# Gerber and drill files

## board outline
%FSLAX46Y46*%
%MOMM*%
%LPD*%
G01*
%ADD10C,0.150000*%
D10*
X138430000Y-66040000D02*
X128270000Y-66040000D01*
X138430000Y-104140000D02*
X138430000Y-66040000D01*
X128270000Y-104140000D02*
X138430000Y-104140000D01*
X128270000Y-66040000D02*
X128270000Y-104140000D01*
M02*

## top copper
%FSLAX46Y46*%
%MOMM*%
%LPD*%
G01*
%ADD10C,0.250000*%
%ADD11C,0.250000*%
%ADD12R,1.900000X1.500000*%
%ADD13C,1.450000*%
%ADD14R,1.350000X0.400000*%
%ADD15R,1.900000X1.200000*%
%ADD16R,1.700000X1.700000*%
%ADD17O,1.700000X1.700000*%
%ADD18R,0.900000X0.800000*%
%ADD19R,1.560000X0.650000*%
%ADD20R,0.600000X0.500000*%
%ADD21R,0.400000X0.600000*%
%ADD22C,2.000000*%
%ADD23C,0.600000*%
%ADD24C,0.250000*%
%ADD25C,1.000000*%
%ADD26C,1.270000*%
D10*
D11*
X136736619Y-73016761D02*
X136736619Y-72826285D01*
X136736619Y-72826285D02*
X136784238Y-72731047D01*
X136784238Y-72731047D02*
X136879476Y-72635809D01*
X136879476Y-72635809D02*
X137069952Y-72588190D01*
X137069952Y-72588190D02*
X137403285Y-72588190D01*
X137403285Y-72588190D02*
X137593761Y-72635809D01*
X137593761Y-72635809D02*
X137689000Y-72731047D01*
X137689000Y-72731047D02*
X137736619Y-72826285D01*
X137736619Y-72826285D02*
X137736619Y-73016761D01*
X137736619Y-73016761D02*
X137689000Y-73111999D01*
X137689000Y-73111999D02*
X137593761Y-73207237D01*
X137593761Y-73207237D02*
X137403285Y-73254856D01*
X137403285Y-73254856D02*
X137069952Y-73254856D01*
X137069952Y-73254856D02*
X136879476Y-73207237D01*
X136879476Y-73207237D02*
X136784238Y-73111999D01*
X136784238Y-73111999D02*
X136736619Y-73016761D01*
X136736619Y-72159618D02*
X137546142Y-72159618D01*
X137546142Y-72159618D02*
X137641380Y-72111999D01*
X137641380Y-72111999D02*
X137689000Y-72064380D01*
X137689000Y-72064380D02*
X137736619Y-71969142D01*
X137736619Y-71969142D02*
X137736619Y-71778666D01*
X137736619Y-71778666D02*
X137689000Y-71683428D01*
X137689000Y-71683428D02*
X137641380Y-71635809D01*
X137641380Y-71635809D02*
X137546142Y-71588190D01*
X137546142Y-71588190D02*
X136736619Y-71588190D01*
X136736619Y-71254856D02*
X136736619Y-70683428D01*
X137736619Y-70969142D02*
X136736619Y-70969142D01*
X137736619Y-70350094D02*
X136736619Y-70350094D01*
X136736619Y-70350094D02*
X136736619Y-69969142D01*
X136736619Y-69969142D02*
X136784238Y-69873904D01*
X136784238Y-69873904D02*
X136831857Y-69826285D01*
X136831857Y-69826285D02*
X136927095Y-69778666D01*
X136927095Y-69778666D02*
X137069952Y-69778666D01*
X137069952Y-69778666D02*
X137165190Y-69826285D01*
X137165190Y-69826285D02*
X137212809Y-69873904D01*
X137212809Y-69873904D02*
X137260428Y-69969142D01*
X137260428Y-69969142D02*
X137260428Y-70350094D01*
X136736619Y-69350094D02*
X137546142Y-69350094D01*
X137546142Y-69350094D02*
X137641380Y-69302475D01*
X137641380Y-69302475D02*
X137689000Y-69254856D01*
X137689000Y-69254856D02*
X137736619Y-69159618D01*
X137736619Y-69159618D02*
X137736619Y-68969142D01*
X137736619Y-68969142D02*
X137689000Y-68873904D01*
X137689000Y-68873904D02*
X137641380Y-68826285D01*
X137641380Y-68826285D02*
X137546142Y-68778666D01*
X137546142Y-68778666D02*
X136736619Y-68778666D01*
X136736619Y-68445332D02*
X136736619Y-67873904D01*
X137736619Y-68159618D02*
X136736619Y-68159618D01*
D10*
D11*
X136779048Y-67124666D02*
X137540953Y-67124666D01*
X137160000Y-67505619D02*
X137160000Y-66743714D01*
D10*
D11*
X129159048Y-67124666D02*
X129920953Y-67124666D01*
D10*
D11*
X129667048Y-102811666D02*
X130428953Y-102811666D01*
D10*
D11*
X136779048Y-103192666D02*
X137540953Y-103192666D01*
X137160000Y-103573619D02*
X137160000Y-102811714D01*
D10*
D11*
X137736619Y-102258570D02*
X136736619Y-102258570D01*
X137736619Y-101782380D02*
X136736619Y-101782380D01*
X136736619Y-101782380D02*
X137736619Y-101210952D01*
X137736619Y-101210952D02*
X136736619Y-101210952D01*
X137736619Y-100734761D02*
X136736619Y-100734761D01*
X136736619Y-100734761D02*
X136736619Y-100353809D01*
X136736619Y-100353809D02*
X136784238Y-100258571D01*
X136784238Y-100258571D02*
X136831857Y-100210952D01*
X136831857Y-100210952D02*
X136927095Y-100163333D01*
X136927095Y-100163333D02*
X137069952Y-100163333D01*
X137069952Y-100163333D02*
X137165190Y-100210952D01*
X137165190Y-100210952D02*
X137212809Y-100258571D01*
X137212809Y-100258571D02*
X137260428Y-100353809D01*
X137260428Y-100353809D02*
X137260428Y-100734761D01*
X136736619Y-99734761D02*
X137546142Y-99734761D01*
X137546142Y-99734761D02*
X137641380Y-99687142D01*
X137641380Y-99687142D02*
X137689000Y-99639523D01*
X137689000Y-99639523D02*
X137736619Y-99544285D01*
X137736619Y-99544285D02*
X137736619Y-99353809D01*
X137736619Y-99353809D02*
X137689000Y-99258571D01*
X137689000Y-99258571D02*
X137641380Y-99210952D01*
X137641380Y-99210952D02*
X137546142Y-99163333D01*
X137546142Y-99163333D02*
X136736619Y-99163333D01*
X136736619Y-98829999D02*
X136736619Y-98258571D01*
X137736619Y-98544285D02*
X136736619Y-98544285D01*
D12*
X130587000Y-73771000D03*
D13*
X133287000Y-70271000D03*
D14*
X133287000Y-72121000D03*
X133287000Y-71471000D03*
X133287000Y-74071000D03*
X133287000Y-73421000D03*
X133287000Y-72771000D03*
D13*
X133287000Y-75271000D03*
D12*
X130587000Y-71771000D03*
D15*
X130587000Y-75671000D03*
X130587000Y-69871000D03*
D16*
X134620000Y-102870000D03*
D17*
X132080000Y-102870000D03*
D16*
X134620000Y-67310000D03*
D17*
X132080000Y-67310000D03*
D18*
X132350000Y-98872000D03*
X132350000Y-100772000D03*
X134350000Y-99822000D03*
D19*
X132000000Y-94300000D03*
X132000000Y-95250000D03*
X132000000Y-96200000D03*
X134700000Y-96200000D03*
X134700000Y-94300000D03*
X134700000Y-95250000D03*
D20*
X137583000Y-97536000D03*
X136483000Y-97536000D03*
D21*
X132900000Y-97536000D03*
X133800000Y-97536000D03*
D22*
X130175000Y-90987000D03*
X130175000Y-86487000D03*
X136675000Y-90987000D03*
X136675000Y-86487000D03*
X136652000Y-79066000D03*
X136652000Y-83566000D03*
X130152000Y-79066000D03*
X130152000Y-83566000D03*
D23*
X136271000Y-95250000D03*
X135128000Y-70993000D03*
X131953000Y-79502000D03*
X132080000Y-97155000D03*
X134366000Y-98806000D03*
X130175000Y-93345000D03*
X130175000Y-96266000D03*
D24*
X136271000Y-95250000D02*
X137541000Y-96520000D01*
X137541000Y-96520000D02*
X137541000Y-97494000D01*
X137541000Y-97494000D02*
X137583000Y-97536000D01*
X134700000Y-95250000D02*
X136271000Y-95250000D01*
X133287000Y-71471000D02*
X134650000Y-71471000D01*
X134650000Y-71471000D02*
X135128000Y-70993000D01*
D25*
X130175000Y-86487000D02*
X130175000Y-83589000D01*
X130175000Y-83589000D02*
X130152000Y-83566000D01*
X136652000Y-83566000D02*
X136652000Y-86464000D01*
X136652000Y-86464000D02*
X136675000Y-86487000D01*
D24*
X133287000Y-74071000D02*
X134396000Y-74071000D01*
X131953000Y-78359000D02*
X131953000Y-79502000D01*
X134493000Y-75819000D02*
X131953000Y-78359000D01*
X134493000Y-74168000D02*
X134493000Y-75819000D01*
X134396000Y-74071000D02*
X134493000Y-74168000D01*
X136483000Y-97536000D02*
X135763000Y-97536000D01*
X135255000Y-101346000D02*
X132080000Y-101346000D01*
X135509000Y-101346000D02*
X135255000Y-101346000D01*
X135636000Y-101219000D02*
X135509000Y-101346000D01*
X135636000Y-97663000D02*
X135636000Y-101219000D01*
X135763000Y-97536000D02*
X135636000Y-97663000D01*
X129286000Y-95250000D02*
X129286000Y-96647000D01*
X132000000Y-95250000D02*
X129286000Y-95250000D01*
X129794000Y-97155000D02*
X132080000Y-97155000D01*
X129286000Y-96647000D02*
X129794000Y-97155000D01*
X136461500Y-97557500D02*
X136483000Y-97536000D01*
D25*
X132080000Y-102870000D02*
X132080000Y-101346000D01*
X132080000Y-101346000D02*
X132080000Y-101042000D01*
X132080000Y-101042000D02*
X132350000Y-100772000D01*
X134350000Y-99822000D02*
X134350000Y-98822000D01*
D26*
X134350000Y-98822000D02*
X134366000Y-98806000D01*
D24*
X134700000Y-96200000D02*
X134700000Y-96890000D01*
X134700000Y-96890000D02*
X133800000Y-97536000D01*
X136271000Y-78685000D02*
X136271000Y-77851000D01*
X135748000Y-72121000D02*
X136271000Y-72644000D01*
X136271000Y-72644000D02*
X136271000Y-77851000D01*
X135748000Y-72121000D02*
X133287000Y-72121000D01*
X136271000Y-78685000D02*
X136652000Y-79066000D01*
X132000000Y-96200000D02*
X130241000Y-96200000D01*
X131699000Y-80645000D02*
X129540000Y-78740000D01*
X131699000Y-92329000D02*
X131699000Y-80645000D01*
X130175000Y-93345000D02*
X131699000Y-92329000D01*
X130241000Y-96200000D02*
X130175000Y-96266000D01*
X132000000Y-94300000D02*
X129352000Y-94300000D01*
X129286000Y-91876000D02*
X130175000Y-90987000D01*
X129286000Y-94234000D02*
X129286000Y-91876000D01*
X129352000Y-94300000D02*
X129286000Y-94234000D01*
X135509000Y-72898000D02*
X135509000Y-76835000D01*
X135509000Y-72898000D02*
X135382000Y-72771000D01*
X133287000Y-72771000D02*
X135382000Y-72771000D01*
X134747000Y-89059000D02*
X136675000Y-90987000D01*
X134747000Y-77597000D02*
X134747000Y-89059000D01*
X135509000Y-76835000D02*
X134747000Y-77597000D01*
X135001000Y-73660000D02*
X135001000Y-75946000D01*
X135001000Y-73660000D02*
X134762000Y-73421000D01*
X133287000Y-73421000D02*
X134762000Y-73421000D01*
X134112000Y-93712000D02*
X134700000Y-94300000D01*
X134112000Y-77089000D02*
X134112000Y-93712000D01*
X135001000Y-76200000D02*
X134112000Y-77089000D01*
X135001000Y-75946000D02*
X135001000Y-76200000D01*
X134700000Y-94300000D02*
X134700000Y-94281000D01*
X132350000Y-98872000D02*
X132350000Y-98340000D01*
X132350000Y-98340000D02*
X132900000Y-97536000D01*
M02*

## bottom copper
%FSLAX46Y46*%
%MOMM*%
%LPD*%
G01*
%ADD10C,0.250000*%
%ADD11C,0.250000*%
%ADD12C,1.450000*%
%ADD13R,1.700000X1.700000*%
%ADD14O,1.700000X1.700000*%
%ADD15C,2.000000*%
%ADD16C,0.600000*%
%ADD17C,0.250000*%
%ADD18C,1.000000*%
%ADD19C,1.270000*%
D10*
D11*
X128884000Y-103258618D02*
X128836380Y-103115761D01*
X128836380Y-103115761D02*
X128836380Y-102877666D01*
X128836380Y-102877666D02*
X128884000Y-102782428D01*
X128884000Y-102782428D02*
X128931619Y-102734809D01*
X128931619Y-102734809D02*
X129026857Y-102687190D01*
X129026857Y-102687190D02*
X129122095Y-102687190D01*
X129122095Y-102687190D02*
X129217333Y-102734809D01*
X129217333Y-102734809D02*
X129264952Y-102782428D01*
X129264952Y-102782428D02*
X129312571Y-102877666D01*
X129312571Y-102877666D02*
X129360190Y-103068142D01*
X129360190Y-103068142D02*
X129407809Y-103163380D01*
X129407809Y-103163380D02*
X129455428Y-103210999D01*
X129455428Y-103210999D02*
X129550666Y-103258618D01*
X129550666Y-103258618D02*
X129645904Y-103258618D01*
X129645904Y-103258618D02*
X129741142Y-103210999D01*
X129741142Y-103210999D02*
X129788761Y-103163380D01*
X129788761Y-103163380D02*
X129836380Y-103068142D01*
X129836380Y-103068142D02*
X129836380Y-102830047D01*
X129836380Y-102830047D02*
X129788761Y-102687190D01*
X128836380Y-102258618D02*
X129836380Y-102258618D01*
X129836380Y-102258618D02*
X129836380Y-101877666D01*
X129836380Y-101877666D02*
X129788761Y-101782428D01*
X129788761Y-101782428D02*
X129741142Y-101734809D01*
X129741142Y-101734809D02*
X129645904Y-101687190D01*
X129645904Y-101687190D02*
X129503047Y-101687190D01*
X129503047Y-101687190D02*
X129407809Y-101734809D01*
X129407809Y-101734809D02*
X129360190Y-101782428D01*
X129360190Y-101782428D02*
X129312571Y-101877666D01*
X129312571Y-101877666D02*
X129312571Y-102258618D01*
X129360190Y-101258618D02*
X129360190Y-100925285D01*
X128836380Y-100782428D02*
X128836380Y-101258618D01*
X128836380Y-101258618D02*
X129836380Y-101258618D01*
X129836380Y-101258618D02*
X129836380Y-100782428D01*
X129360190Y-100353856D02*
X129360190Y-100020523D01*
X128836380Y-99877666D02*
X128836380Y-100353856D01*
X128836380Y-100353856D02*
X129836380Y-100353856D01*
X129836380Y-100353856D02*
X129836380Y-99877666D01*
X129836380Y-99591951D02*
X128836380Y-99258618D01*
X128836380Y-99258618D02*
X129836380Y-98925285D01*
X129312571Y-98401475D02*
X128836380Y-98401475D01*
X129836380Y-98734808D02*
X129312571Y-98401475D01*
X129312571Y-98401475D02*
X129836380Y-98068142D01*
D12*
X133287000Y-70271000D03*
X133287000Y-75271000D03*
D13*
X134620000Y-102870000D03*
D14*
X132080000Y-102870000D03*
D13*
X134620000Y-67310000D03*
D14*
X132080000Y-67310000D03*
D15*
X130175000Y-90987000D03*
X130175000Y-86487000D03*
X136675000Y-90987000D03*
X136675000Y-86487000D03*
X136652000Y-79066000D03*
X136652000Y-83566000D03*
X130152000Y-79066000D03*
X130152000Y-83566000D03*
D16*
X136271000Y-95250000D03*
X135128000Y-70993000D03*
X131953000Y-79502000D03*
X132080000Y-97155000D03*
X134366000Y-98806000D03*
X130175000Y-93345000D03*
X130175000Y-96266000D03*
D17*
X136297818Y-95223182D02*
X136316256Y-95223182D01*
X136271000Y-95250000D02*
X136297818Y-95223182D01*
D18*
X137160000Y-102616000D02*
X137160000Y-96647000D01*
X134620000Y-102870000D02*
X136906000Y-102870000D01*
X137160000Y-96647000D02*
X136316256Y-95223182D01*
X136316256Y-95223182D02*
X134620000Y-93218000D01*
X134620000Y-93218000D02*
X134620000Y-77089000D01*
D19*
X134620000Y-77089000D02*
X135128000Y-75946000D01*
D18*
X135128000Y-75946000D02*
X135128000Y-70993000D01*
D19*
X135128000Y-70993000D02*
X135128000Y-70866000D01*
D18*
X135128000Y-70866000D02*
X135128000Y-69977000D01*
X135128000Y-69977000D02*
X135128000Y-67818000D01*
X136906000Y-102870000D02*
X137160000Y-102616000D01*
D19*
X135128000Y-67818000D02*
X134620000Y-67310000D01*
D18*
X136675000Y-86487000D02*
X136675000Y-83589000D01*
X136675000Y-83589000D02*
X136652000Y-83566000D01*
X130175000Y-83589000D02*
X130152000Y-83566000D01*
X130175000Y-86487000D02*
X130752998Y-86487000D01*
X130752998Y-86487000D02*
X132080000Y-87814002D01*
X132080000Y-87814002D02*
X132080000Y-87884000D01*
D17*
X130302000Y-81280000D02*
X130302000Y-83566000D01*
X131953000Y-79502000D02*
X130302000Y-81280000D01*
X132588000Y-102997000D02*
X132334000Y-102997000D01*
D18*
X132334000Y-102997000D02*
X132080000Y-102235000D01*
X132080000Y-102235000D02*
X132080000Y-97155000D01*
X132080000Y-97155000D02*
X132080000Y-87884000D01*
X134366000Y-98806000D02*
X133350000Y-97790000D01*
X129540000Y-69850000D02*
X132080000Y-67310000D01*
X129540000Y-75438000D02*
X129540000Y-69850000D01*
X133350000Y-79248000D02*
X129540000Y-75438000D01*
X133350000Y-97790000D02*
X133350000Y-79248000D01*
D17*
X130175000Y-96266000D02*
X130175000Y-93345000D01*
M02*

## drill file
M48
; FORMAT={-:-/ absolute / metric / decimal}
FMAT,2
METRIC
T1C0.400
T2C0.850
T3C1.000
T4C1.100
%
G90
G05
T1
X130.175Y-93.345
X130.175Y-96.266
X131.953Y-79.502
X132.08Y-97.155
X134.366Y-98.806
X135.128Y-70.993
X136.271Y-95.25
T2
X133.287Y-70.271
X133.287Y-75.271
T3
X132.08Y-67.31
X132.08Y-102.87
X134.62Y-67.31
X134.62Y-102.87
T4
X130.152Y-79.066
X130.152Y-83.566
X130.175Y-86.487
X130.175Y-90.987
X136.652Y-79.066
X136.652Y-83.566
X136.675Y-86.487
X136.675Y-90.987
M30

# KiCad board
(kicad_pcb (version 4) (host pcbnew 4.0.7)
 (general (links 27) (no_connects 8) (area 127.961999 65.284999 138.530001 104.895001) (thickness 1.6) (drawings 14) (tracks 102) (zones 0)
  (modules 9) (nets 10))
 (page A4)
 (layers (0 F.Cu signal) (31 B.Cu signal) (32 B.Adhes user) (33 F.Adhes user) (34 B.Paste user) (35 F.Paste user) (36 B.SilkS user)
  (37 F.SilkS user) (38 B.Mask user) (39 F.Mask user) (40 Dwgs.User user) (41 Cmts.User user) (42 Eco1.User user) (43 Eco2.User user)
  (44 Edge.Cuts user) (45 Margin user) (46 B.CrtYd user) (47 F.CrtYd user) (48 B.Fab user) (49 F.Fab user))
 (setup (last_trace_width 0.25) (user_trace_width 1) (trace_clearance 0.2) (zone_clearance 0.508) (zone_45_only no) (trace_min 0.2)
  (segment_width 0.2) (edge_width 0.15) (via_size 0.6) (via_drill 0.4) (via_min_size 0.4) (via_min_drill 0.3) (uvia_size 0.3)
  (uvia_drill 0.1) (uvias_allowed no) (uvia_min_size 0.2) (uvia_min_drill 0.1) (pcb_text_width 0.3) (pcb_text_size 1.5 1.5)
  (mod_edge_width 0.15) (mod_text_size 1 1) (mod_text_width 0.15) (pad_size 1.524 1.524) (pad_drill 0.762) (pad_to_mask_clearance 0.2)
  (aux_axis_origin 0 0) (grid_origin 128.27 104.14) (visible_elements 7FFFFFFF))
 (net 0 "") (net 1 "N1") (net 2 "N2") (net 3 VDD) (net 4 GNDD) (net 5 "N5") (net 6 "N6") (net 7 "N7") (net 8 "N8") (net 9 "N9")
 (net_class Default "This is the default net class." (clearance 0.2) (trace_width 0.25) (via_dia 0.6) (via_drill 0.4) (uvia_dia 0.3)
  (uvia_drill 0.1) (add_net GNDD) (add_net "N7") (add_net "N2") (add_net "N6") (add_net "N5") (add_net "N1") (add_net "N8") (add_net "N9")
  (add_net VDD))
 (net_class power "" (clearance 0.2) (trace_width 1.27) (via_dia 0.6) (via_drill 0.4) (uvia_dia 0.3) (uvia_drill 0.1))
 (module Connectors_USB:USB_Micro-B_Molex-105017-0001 (layer F.Cu) (at 130.937 72.771 270)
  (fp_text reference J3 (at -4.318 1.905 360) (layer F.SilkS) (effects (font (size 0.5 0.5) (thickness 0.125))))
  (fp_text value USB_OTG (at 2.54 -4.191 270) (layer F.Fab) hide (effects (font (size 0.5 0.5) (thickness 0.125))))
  (pad 6 smd rect (at 1 0.35 270) (size 1.5 1.9) (layers F.Cu F.Paste F.Mask) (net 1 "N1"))
  (pad 6 thru_hole circle (at -2.5 -2.35 270) (size 1.45 1.45) (drill 0.85) (layers *.Cu *.Mask) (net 1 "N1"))
  (pad 2 smd rect (at -0.65 -2.35 270) (size 0.4 1.35) (layers F.Cu F.Paste F.Mask) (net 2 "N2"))
  (pad 1 smd rect (at -1.3 -2.35 270) (size 0.4 1.35) (layers F.Cu F.Paste F.Mask) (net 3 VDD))
  (pad 5 smd rect (at 1.3 -2.35 270) (size 0.4 1.35) (layers F.Cu F.Paste F.Mask) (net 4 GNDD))
  (pad 4 smd rect (at 0.65 -2.35 270) (size 0.4 1.35) (layers F.Cu F.Paste F.Mask) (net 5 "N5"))
  (pad 3 smd rect (at 0 -2.35 270) (size 0.4 1.35) (layers F.Cu F.Paste F.Mask) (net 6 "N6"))
  (pad 6 thru_hole circle (at 2.5 -2.35 270) (size 1.45 1.45) (drill 0.85) (layers *.Cu *.Mask) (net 1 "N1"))
  (pad 6 smd rect (at -1 0.35 270) (size 1.5 1.9) (layers F.Cu F.Paste F.Mask) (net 1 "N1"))
  (pad 6 smd rect (at 2.9 0.35 270) (size 1.2 1.9) (layers F.Cu F.Mask) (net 1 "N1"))
  (pad 6 smd rect (at -2.9 0.35 270) (size 1.2 1.9) (layers F.Cu F.Mask) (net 1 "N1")))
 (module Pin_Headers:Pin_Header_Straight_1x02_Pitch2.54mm (layer F.Cu) (at 134.62 102.87 270)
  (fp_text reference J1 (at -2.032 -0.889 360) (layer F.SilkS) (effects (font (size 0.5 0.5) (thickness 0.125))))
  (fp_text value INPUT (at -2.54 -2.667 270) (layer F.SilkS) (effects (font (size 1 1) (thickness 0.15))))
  (pad 1 thru_hole rect (at 0 0 270) (size 1.7 1.7) (drill 1) (layers *.Cu *.Mask) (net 3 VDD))
  (pad 2 thru_hole oval (at 0 2.54 270) (size 1.7 1.7) (drill 1) (layers *.Cu *.Mask) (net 4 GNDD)))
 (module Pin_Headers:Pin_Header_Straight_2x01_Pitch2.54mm (layer F.Cu) (at 134.62 67.31 180)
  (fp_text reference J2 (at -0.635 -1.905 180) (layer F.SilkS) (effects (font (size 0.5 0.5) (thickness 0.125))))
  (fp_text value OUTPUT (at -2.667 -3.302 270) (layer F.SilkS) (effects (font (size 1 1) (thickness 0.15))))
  (pad 1 thru_hole rect (at 0 0 180) (size 1.7 1.7) (drill 1) (layers *.Cu *.Mask) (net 3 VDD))
  (pad 2 thru_hole oval (at 2.54 0 180) (size 1.7 1.7) (drill 1) (layers *.Cu *.Mask) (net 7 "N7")))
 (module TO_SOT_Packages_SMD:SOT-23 (layer F.Cu) (at 133.35 99.822)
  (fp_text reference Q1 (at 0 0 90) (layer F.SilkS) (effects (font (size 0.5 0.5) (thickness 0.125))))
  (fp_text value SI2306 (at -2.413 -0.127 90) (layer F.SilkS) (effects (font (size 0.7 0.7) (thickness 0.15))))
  (pad 1 smd rect (at -1 -0.95) (size 0.9 0.8) (layers F.Cu F.Paste F.Mask) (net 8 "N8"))
  (pad 2 smd rect (at -1 0.95) (size 0.9 0.8) (layers F.Cu F.Paste F.Mask) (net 4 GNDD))
  (pad 3 smd rect (at 1 0) (size 0.9 0.8) (layers F.Cu F.Paste F.Mask) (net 7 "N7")))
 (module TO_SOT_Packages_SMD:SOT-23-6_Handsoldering (layer F.Cu) (at 133.35 95.25)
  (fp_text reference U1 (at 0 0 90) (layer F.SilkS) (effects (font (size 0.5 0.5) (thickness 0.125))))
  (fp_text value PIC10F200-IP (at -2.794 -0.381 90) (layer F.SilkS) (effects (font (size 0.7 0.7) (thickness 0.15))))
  (pad 1 smd rect (at -1.35 -0.95) (size 1.56 0.65) (layers F.Cu F.Paste F.Mask) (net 6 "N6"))
  (pad 2 smd rect (at -1.35 0) (size 1.56 0.65) (layers F.Cu F.Paste F.Mask) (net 4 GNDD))
  (pad 3 smd rect (at -1.35 0.95) (size 1.56 0.65) (layers F.Cu F.Paste F.Mask) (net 2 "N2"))
  (pad 4 smd rect (at 1.35 0.95) (size 1.56 0.65) (layers F.Cu F.Paste F.Mask) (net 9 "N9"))
  (pad 6 smd rect (at 1.35 -0.95) (size 1.56 0.65) (layers F.Cu F.Paste F.Mask) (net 5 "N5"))
  (pad 5 smd rect (at 1.35 0) (size 1.56 0.65) (layers F.Cu F.Paste F.Mask) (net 3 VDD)))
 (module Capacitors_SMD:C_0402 (layer F.Cu) (at 137.033 97.536 180)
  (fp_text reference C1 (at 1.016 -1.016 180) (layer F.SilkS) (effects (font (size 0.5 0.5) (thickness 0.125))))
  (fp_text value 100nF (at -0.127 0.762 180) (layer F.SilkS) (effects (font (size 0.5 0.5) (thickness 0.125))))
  (pad 1 smd rect (at -0.55 0 180) (size 0.6 0.5) (layers F.Cu F.Paste F.Mask) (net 3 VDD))
  (pad 2 smd rect (at 0.55 0 180) (size 0.6 0.5) (layers F.Cu F.Paste F.Mask) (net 4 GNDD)))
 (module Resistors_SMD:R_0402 (layer F.Cu) (at 133.35 97.536)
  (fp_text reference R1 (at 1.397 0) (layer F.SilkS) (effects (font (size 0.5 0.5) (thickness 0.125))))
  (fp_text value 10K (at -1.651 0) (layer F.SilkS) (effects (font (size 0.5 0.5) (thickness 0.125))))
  (pad 1 smd rect (at -0.45 0) (size 0.4 0.6) (layers F.Cu F.Paste F.Mask) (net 8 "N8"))
  (pad 2 smd rect (at 0.45 0) (size 0.4 0.6) (layers F.Cu F.Paste F.Mask) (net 9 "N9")))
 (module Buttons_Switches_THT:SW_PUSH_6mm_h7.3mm (layer F.Cu) (at 130.175 86.487)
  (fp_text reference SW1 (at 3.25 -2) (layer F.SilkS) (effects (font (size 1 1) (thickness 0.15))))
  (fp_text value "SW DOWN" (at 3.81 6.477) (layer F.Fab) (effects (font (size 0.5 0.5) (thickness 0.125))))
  (pad 2 thru_hole circle (at 0 4.5 90) (size 2 2) (drill 1.1) (layers *.Cu *.Mask) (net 6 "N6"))
  (pad 1 thru_hole circle (at 0 0 90) (size 2 2) (drill 1.1) (layers *.Cu *.Mask) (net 4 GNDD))
  (pad 2 thru_hole circle (at 6.5 4.5 90) (size 2 2) (drill 1.1) (layers *.Cu *.Mask) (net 6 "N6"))
  (pad 1 thru_hole circle (at 6.5 0 90) (size 2 2) (drill 1.1) (layers *.Cu *.Mask) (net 4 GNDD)))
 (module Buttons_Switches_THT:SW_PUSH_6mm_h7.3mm (layer F.Cu) (at 136.652 83.566 180)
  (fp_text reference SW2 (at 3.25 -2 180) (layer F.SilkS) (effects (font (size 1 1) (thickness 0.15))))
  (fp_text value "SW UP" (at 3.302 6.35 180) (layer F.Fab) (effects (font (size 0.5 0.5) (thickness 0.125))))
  (pad 2 thru_hole circle (at 0 4.5 270) (size 2 2) (drill 1.1) (layers *.Cu *.Mask) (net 2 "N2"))
  (pad 1 thru_hole circle (at 0 0 270) (size 2 2) (drill 1.1) (layers *.Cu *.Mask) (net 4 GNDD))
  (pad 2 thru_hole circle (at 6.5 4.5 270) (size 2 2) (drill 1.1) (layers *.Cu *.Mask) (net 2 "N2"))
  (pad 1 thru_hole circle (at 6.5 0 270) (size 2 2) (drill 1.1) (layers *.Cu *.Mask) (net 4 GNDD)))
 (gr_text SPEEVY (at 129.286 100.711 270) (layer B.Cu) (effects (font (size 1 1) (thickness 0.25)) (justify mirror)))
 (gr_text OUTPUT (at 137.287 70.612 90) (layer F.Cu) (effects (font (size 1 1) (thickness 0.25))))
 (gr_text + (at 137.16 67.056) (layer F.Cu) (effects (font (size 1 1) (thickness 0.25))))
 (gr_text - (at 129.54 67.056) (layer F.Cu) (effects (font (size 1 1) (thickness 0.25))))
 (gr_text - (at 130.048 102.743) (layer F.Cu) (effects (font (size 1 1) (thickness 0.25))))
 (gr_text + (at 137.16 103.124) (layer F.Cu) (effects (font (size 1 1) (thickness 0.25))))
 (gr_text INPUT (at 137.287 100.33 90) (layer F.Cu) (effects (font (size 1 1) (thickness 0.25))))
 (gr_line (start 138.43 66.04) (end 128.27 66.04) (angle 90) (layer Edge.Cuts) (width 0.15))
 (gr_line (start 138.43 104.14) (end 138.43 66.04) (angle 90) (layer Edge.Cuts) (width 0.15))
 (gr_line (start 128.27 104.14) (end 138.43 104.14) (angle 90) (layer Edge.Cuts) (width 0.15))
 (gr_line (start 128.27 66.04) (end 128.27 104.14) (angle 90) (layer Edge.Cuts) (width 0.15))
 (segment (start 136.271 95.25) (end 137.541 96.52) (width 0.25) (layer F.Cu) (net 3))
 (segment (start 137.541 96.52) (end 137.541 97.494) (width 0.25) (layer F.Cu) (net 3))
 (segment (start 137.541 97.494) (end 137.583 97.536) (width 0.25) (layer F.Cu) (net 3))
 (segment (start 134.7 95.25) (end 136.271 95.25) (width 0.25) (layer F.Cu) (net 3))
 (segment (start 136.297818 95.223182) (end 136.316256 95.223182) (width 0.25) (layer B.Cu) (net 3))
 (segment (start 136.271 95.25) (end 136.297818 95.223182) (width 0.25) (layer B.Cu) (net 3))
 (via (at 136.271 95.25) (size 0.6) (drill 0.4) (layers F.Cu B.Cu) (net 3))
 (segment (start 133.287 71.471) (end 134.65 71.471) (width 0.25) (layer F.Cu) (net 3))
 (via (at 135.128 70.993) (size 0.6) (drill 0.4) (layers F.Cu B.Cu) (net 3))
 (segment (start 134.65 71.471) (end 135.128 70.993) (width 0.25) (layer F.Cu) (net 3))
 (segment (start 137.16 102.616) (end 137.16 96.647) (width 1) (layer B.Cu) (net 3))
 (segment (start 134.62 102.87) (end 136.906 102.87) (width 1) (layer B.Cu) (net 3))
 (segment (start 137.16 96.647) (end 136.316256 95.223182) (width 1) (layer B.Cu) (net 3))
 (segment (start 136.316256 95.223182) (end 134.62 93.218) (width 1) (layer B.Cu) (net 3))
 (segment (start 134.62 93.218) (end 134.62 77.089) (width 1) (layer B.Cu) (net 3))
 (segment (start 134.62 77.089) (end 135.128 75.946) (width 1.27) (layer B.Cu) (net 3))
 (segment (start 135.128 75.946) (end 135.128 70.993) (width 1) (layer B.Cu) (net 3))
 (segment (start 135.128 70.993) (end 135.128 70.866) (width 1.27) (layer B.Cu) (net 3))
 (segment (start 135.128 70.866) (end 135.128 69.977) (width 1) (layer B.Cu) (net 3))
 (segment (start 135.128 69.977) (end 135.128 67.818) (width 1) (layer B.Cu) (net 3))
 (segment (start 136.906 102.87) (end 137.16 102.616) (width 1) (layer B.Cu) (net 3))
 (segment (start 135.128 67.818) (end 134.62 67.31) (width 1.27) (layer B.Cu) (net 3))
 (segment (start 130.175 86.487) (end 130.175 83.589) (width 1) (layer F.Cu) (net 4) (status C00000))
 (segment (start 130.175 83.589) (end 130.152 83.566) (width 1) (layer F.Cu) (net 4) (status C00000))
 (segment (start 136.652 83.566) (end 136.652 86.464) (width 1) (layer F.Cu) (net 4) (status C00000))
 (segment (start 136.652 86.464) (end 136.675 86.487) (width 1) (layer F.Cu) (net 4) (status C00000))
 (segment (start 136.675 86.487) (end 136.675 83.589) (width 1) (layer B.Cu) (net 4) (status C00000))
 (segment (start 136.675 83.589) (end 136.652 83.566) (width 1) (layer B.Cu) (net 4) (status C00000))
 (segment (start 130.175 83.589) (end 130.152 83.566) (width 1) (layer B.Cu) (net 4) (status C00000))
 (segment (start 130.175 86.487) (end 130.752998 86.487) (width 1) (layer B.Cu) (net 4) (status C00000))
 (segment (start 130.752998 86.487) (end 132.08 87.814002) (width 1) (layer B.Cu) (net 4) (status 400000))
 (segment (start 132.08 87.814002) (end 132.08 87.884) (width 1) (layer B.Cu) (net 4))
 (segment (start 133.287 74.071) (end 134.396 74.071) (width 0.25) (layer F.Cu) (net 4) (status 400000))
 (segment (start 130.302 81.28) (end 130.302 83.566) (width 0.25) (layer B.Cu) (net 4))
 (segment (start 131.953 79.502) (end 130.302 81.28) (width 0.25) (layer B.Cu) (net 4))
 (via (at 131.953 79.502) (size 0.6) (drill 0.4) (layers F.Cu B.Cu) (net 4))
 (segment (start 131.953 78.359) (end 131.953 79.502) (width 0.25) (layer F.Cu) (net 4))
 (segment (start 134.493 75.819) (end 131.953 78.359) (width 0.25) (layer F.Cu) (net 4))
 (segment (start 134.493 74.168) (end 134.493 75.819) (width 0.25) (layer F.Cu) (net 4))
 (segment (start 134.396 74.071) (end 134.493 74.168) (width 0.25) (layer F.Cu) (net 4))
 (segment (start 136.483 97.536) (end 135.763 97.536) (width 0.25) (layer F.Cu) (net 4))
 (segment (start 135.255 101.346) (end 132.08 101.346) (width 0.25) (layer F.Cu) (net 4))
 (segment (start 135.509 101.346) (end 135.255 101.346) (width 0.25) (layer F.Cu) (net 4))
 (segment (start 135.636 101.219) (end 135.509 101.346) (width 0.25) (layer F.Cu) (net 4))
 (segment (start 135.636 97.663) (end 135.636 101.219) (width 0.25) (layer F.Cu) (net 4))
 (segment (start 135.763 97.536) (end 135.636 97.663) (width 0.25) (layer F.Cu) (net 4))
 (segment (start 129.286 95.25) (end 129.286 96.647) (width 0.25) (layer F.Cu) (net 4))
 (segment (start 132 95.25) (end 129.286 95.25) (width 0.25) (layer F.Cu) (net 4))
 (via (at 132.08 97.155) (size 0.6) (drill 0.4) (layers F.Cu B.Cu) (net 4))
 (segment (start 129.794 97.155) (end 132.08 97.155) (width 0.25) (layer F.Cu) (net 4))
 (segment (start 129.286 96.647) (end 129.794 97.155) (width 0.25) (layer F.Cu) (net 4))
 (segment (start 132.588 102.997) (end 132.334 102.997) (width 0.25) (layer B.Cu) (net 4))
 (segment (start 132.334 102.997) (end 132.08 102.235) (width 1) (layer B.Cu) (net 4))
 (segment (start 132.08 102.235) (end 132.08 97.155) (width 1) (layer B.Cu) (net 4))
 (segment (start 132.08 97.155) (end 132.08 87.884) (width 1) (layer B.Cu) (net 4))
 (segment (start 136.4615 97.5575) (end 136.483 97.536) (width 0.25) (layer F.Cu) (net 4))
 (segment (start 132.08 102.87) (end 132.08 101.346) (width 1) (layer F.Cu) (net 4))
 (segment (start 132.08 101.346) (end 132.08 101.042) (width 1) (layer F.Cu) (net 4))
 (segment (start 132.08 101.042) (end 132.35 100.772) (width 1) (layer F.Cu) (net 4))
 (segment (start 134.366 98.806) (end 133.35 97.79) (width 1) (layer B.Cu) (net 7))
 (segment (start 134.35 99.822) (end 134.35 98.822) (width 1) (layer F.Cu) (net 7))
 (via (at 134.366 98.806) (size 0.6) (drill 0.4) (layers F.Cu B.Cu) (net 7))
 (segment (start 134.35 98.822) (end 134.366 98.806) (width 1.27) (layer F.Cu) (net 7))
 (segment (start 129.54 69.85) (end 132.08 67.31) (width 1) (layer B.Cu) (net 7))
 (segment (start 129.54 75.438) (end 129.54 69.85) (width 1) (layer B.Cu) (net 7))
 (segment (start 133.35 79.248) (end 129.54 75.438) (width 1) (layer B.Cu) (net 7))
 (segment (start 133.35 97.79) (end 133.35 79.248) (width 1) (layer B.Cu) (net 7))
 (segment (start 134.7 96.2) (end 134.7 96.89) (width 0.25) (layer F.Cu) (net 9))
 (segment (start 134.7 96.89) (end 133.8 97.536) (width 0.25) (layer F.Cu) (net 9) (status 20))
 (segment (start 136.271 78.685) (end 136.271 77.851) (width 0.25) (layer F.Cu) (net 2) (status 400000))
 (segment (start 135.748 72.121) (end 136.271 72.644) (width 0.25) (layer F.Cu) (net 2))
 (segment (start 136.271 72.644) (end 136.271 77.851) (width 0.25) (layer F.Cu) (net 2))
 (segment (start 135.748 72.121) (end 133.287 72.121) (width 0.25) (layer F.Cu) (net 2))
 (segment (start 136.271 78.685) (end 136.652 79.066) (width 0.25) (layer F.Cu) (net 2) (status C00000))
 (segment (start 132 96.2) (end 130.241 96.2) (width 0.25) (layer F.Cu) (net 2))
 (segment (start 131.699 80.645) (end 129.54 78.74) (width 0.25) (layer F.Cu) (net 2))
 (segment (start 131.699 92.329) (end 131.699 80.645) (width 0.25) (layer F.Cu) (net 2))
 (segment (start 130.175 93.345) (end 131.699 92.329) (width 0.25) (layer F.Cu) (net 2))
 (via (at 130.175 93.345) (size 0.6) (drill 0.4) (layers F.Cu B.Cu) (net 2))
 (segment (start 130.175 96.266) (end 130.175 93.345) (width 0.25) (layer B.Cu) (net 2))
 (via (at 130.175 96.266) (size 0.6) (drill 0.4) (layers F.Cu B.Cu) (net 2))
 (segment (start 130.241 96.2) (end 130.175 96.266) (width 0.25) (layer F.Cu) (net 2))
 (segment (start 132 94.3) (end 129.352 94.3) (width 0.25) (layer F.Cu) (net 6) (status 400000))
 (segment (start 129.286 91.876) (end 130.175 90.987) (width 0.25) (layer F.Cu) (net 6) (status 800000))
 (segment (start 129.286 94.234) (end 129.286 91.876) (width 0.25) (layer F.Cu) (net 6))
 (segment (start 129.352 94.3) (end 129.286 94.234) (width 0.25) (layer F.Cu) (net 6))
 (segment (start 135.509 72.898) (end 135.509 76.835) (width 0.25) (layer F.Cu) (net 6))
 (segment (start 135.509 72.898) (end 135.382 72.771) (width 0.25) (layer F.Cu) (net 6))
 (segment (start 133.287 72.771) (end 135.382 72.771) (width 0.25) (layer F.Cu) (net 6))
 (segment (start 134.747 89.059) (end 136.675 90.987) (width 0.25) (layer F.Cu) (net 6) (status 800000))
 (segment (start 134.747 77.597) (end 134.747 89.059) (width 0.25) (layer F.Cu) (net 6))
 (segment (start 135.509 76.835) (end 134.747 77.597) (width 0.25) (layer F.Cu) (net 6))
 (segment (start 135.001 73.66) (end 135.001 75.946) (width 0.25) (layer F.Cu) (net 5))
 (segment (start 135.001 73.66) (end 134.762 73.421) (width 0.25) (layer F.Cu) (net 5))
 (segment (start 133.287 73.421) (end 134.762 73.421) (width 0.25) (layer F.Cu) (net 5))
 (segment (start 134.112 93.712) (end 134.7 94.3) (width 0.25) (layer F.Cu) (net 5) (status 800000))
 (segment (start 134.112 77.089) (end 134.112 93.712) (width 0.25) (layer F.Cu) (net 5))
 (segment (start 135.001 76.2) (end 134.112 77.089) (width 0.25) (layer F.Cu) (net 5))
 (segment (start 135.001 75.946) (end 135.001 76.2) (width 0.25) (layer F.Cu) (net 5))
 (segment (start 134.7 94.3) (end 134.7 94.281) (width 0.25) (layer F.Cu) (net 5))
 (segment (start 132.35 98.872) (end 132.35 98.34) (width 0.25) (layer F.Cu) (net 8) (status 10))
 (segment (start 132.35 98.34) (end 132.9 97.536) (width 0.25) (layer F.Cu) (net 8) (status 20)))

